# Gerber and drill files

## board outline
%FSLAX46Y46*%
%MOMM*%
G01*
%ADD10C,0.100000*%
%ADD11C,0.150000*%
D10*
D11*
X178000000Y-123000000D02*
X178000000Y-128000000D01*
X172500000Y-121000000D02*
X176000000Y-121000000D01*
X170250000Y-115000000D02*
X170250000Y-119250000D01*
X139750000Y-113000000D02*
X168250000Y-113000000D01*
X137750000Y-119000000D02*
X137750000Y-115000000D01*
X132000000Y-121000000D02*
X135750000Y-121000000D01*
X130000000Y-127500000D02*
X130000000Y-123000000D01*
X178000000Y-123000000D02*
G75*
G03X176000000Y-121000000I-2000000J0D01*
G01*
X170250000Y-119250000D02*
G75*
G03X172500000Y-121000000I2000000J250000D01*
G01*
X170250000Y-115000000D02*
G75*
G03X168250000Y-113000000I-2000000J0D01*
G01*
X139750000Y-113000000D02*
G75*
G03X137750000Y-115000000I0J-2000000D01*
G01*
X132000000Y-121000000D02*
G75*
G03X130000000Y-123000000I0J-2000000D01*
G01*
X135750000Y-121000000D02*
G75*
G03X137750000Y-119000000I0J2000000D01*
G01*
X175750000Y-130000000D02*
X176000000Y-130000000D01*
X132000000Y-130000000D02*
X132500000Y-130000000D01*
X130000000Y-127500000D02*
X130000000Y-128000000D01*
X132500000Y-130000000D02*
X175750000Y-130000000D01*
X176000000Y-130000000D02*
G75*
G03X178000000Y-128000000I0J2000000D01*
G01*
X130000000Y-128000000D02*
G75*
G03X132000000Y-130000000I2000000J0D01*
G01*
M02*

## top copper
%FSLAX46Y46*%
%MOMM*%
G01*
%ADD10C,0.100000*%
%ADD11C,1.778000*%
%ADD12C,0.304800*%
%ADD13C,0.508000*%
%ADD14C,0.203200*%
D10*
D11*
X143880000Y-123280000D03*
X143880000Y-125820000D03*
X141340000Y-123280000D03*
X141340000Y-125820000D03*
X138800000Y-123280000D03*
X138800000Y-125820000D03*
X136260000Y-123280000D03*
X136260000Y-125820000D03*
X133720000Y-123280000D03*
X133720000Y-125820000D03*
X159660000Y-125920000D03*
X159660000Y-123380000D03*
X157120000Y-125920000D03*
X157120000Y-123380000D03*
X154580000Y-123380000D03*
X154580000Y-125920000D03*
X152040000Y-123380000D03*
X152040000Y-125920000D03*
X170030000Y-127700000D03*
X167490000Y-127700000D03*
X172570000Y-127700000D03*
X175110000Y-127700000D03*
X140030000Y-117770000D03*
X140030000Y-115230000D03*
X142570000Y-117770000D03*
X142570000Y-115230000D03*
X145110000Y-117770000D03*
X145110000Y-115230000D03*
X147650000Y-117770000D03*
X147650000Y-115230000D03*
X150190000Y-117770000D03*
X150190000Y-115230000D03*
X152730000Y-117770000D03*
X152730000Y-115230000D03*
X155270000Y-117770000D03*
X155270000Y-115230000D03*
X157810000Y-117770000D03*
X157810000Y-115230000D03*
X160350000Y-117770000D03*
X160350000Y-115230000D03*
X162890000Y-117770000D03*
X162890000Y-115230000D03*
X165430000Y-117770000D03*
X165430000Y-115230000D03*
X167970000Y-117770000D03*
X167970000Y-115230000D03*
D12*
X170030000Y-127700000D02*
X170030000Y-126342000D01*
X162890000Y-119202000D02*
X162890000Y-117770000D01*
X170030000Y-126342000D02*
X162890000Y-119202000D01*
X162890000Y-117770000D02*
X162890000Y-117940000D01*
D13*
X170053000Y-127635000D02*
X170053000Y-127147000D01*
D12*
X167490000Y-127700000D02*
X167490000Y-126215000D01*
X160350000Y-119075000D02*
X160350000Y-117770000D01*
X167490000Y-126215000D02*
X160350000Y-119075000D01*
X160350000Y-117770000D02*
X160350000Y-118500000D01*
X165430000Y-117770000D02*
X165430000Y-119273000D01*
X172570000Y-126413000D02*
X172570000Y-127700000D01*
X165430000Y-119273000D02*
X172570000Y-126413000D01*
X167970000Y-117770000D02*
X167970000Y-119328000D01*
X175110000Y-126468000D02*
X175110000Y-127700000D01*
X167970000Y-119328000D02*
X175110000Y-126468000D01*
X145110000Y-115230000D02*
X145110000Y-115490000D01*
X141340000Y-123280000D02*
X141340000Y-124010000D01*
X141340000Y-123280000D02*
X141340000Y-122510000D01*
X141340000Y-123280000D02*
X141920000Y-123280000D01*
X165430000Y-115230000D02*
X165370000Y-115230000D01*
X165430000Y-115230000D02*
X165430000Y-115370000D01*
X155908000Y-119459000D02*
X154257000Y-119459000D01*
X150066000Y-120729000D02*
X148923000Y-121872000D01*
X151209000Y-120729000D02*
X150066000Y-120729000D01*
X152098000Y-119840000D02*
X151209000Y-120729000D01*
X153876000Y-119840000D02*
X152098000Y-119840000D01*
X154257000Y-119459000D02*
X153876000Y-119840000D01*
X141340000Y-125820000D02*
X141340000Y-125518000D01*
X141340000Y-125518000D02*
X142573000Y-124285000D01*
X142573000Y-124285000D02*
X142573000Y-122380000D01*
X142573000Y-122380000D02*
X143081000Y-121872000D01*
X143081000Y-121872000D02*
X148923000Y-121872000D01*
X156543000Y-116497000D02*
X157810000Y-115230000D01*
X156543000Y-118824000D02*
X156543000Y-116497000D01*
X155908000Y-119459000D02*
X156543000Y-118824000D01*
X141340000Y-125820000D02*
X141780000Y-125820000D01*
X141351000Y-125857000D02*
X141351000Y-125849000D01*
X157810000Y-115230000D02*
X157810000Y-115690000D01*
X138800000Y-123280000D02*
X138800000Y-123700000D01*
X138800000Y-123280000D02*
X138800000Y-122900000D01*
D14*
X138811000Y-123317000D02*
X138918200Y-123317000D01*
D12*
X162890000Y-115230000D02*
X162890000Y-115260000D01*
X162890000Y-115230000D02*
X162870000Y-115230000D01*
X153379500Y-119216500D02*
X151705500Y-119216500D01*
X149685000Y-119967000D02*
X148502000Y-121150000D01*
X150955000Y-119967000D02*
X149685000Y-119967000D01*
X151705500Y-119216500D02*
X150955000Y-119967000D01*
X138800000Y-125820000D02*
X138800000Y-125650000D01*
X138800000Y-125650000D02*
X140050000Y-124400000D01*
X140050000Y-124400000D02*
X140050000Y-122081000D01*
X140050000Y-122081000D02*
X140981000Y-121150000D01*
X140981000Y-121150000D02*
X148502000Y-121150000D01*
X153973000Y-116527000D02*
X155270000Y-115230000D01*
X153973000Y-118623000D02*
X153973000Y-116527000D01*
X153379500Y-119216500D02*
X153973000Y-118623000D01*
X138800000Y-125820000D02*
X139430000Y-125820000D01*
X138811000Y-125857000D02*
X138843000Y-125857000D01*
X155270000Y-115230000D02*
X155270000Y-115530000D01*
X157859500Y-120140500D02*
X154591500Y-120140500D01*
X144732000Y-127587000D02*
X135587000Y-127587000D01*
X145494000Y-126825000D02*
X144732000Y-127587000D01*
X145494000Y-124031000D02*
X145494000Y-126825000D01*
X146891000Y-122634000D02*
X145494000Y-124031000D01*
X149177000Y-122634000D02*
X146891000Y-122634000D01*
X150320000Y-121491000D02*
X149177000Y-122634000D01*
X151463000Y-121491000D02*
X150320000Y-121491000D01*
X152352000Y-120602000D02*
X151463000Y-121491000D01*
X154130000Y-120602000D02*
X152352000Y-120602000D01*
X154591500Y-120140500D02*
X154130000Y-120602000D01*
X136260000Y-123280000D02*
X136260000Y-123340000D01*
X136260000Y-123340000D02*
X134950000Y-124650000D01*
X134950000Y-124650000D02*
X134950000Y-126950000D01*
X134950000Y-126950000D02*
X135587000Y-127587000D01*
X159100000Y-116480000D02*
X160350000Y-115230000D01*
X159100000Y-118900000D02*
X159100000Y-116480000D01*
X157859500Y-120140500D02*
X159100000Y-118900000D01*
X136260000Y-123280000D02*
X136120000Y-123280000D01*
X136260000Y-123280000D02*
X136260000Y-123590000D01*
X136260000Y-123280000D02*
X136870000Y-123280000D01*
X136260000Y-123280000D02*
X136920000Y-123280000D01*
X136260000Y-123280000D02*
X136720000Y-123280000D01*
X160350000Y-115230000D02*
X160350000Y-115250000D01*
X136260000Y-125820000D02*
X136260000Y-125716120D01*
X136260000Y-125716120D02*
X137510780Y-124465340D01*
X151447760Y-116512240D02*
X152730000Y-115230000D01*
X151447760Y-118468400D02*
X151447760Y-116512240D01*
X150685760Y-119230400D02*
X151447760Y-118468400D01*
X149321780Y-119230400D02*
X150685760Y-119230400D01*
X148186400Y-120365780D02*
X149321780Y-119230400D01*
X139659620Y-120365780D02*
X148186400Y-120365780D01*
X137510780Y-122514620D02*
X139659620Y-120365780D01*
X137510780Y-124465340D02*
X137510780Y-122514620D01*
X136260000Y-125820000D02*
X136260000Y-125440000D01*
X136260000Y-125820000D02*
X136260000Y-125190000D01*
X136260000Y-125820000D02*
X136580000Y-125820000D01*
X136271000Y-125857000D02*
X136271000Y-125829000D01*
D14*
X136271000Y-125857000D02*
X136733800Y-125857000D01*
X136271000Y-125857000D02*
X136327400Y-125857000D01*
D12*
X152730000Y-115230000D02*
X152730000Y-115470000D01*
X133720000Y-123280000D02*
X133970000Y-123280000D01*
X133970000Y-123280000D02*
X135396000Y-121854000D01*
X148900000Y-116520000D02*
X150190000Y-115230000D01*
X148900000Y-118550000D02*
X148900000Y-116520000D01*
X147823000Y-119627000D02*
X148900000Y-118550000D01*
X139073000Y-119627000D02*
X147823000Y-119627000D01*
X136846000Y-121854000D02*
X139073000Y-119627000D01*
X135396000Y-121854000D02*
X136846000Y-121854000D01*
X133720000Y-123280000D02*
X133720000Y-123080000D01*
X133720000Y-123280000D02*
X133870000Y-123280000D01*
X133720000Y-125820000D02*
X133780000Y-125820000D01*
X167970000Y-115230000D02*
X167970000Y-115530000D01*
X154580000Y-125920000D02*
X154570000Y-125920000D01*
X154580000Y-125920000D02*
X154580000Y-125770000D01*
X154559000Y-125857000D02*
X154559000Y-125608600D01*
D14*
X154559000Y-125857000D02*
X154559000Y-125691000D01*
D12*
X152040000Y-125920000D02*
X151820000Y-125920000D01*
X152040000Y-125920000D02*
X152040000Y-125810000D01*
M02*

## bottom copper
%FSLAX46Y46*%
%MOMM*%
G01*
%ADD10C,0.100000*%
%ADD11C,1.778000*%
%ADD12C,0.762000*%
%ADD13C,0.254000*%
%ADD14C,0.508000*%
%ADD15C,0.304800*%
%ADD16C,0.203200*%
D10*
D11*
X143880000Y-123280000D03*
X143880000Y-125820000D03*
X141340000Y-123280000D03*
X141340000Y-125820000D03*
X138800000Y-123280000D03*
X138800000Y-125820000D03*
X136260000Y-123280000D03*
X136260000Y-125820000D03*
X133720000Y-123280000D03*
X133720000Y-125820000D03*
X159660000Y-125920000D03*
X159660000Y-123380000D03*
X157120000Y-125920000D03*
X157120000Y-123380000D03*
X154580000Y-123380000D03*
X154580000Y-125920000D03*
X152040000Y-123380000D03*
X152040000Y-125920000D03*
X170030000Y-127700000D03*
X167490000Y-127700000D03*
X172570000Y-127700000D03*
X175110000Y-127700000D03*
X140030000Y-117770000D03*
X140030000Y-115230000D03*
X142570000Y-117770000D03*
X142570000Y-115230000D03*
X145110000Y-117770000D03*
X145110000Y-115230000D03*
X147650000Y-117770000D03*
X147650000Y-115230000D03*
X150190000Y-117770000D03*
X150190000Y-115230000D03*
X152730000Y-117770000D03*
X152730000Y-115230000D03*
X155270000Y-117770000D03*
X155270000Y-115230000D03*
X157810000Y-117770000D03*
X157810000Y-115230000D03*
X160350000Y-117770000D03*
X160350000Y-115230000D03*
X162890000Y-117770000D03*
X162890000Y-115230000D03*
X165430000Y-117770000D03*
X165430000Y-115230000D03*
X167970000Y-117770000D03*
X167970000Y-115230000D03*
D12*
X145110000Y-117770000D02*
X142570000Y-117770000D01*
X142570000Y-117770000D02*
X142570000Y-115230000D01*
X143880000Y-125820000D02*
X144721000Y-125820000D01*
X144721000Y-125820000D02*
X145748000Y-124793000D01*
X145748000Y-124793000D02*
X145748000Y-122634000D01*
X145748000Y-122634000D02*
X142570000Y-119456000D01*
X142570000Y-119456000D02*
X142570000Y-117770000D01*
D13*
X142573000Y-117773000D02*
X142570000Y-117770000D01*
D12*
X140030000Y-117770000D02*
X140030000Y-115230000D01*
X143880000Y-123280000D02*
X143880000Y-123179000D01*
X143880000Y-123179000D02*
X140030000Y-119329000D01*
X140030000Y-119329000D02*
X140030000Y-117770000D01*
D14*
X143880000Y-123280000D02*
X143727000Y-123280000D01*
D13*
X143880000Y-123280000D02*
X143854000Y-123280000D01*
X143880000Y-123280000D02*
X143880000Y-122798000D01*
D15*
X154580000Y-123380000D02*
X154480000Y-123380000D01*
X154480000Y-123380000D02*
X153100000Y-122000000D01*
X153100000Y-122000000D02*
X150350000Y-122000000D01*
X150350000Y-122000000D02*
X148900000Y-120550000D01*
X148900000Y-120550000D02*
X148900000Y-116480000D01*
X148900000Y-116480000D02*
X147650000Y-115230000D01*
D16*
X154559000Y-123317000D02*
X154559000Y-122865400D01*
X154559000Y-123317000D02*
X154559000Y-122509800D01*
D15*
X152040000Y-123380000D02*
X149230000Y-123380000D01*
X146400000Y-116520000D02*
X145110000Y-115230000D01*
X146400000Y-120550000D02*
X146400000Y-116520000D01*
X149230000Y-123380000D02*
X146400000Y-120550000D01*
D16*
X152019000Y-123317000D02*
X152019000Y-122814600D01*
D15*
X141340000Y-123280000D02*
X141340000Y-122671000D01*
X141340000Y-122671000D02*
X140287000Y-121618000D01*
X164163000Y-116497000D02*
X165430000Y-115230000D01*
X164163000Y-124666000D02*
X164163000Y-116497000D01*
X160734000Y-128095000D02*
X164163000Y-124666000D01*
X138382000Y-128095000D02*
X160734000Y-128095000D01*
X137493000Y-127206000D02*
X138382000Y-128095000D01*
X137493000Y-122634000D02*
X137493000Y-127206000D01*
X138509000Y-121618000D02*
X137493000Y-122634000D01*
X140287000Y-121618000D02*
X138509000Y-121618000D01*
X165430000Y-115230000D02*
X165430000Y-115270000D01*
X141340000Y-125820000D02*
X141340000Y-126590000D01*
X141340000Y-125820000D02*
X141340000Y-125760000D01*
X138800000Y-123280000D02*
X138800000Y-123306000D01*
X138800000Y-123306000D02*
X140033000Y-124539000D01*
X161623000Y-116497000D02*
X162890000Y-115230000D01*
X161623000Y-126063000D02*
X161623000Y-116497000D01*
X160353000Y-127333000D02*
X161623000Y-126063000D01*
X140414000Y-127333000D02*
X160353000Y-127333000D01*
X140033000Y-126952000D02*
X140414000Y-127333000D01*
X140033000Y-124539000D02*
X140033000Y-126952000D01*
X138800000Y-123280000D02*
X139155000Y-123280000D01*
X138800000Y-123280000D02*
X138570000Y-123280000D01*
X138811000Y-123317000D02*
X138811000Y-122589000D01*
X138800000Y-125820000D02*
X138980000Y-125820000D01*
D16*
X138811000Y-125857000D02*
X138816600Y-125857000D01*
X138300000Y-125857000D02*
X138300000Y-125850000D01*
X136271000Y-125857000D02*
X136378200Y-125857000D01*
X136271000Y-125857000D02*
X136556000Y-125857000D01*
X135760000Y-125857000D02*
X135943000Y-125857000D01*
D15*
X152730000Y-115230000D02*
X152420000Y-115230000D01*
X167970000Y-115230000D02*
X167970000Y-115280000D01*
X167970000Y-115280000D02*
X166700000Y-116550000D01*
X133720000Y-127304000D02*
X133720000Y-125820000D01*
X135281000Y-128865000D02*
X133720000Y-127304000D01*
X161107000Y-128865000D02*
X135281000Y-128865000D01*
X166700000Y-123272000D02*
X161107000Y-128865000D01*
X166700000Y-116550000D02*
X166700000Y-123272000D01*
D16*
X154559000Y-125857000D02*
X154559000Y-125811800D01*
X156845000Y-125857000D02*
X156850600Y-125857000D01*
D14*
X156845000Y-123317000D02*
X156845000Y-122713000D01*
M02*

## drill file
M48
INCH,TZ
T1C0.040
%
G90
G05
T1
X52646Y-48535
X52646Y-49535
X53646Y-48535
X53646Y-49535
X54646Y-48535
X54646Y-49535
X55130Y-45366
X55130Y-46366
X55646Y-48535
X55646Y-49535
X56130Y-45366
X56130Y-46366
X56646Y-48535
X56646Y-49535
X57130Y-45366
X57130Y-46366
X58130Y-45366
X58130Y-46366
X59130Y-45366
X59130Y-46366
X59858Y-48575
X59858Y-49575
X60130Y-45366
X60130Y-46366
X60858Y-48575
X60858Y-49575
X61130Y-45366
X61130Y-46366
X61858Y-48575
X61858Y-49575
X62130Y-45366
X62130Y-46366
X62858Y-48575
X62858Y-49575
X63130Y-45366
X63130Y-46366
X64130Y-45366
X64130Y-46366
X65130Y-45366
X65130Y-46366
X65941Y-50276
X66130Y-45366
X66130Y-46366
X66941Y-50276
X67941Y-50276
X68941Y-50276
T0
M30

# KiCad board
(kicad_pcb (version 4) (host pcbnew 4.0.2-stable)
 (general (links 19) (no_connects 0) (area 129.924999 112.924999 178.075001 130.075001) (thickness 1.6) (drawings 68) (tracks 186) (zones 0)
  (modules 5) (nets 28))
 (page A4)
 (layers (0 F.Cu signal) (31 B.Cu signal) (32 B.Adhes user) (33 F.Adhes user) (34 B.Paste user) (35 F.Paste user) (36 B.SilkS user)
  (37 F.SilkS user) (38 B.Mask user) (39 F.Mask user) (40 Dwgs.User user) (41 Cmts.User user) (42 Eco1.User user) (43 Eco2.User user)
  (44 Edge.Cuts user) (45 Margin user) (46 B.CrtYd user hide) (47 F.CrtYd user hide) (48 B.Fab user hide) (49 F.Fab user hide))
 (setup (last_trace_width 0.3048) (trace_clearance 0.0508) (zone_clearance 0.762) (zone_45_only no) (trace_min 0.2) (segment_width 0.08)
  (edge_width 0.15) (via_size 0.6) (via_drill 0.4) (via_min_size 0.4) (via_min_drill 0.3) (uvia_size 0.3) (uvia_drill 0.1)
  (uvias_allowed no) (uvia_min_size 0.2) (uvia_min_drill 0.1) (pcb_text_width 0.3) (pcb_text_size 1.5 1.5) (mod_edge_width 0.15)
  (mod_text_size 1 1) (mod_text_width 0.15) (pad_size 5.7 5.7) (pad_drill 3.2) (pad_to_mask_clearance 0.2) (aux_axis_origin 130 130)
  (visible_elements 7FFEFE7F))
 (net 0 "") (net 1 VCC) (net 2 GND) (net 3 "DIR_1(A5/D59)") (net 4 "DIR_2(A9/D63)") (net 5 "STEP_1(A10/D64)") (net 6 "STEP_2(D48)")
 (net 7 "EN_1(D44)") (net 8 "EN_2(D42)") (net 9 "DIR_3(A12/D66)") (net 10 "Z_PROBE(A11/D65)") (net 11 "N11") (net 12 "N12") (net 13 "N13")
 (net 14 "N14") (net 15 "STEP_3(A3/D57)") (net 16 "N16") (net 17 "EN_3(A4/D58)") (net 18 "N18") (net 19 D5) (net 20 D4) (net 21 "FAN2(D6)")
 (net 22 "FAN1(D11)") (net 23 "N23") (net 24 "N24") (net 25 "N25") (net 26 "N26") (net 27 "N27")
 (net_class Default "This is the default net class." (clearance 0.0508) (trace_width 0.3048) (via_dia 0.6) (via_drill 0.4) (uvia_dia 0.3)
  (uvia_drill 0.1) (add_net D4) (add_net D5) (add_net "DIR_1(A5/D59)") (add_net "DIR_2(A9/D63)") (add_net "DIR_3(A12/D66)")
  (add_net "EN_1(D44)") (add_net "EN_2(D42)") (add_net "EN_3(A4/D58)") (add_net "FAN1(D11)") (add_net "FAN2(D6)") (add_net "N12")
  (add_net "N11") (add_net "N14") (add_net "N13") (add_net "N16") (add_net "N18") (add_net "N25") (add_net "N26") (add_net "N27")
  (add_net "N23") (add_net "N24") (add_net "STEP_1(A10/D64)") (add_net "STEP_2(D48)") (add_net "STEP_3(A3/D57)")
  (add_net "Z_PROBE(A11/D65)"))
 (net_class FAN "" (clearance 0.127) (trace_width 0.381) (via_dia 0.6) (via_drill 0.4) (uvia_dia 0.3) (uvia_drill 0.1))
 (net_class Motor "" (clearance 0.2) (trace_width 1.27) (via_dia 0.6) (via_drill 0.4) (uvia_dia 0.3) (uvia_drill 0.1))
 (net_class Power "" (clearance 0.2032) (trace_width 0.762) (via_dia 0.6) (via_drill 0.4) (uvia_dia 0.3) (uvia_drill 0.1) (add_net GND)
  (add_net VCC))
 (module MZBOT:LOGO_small (layer F.Cu) (at 167.66058 124.78538)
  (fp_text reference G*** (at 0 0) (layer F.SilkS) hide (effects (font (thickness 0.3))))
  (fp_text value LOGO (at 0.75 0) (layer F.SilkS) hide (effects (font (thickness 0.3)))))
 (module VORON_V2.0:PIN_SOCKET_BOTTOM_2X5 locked (layer F.Cu) (at 138.8 124.55 180)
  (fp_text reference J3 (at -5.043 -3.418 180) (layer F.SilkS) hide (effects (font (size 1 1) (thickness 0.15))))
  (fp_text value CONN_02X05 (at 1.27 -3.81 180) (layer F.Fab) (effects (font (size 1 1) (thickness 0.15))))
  (pad 1 thru_hole circle (at -5.08 1.27 180) (size 1.778 1.778) (drill 1.016) (layers *.Cu *.Mask F.SilkS) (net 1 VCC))
  (pad 2 thru_hole circle (at -5.08 -1.27 180) (size 1.778 1.778) (drill 1.016) (layers *.Cu *.Mask F.SilkS) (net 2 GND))
  (pad 3 thru_hole circle (at -2.54 1.27 180) (size 1.778 1.778) (drill 1.016) (layers *.Cu *.Mask F.SilkS) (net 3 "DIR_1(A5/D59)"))
  (pad 4 thru_hole circle (at -2.54 -1.27 180) (size 1.778 1.778) (drill 1.016) (layers *.Cu *.Mask F.SilkS) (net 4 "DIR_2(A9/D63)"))
  (pad 5 thru_hole circle (at 0 1.27 180) (size 1.778 1.778) (drill 1.016) (layers *.Cu *.Mask F.SilkS) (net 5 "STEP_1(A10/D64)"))
  (pad 6 thru_hole circle (at 0 -1.27 180) (size 1.778 1.778) (drill 1.016) (layers *.Cu *.Mask F.SilkS) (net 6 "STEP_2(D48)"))
  (pad 7 thru_hole circle (at 2.54 1.27 180) (size 1.778 1.778) (drill 1.016) (layers *.Cu *.Mask F.SilkS) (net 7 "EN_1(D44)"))
  (pad 8 thru_hole circle (at 2.54 -1.27 180) (size 1.778 1.778) (drill 1.016) (layers *.Cu *.Mask F.SilkS) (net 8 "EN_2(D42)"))
  (pad 9 thru_hole circle (at 5.08 1.27 180) (size 1.778 1.778) (drill 1.016) (layers *.Cu *.Mask F.SilkS) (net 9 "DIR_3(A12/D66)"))
  (pad 10 thru_hole circle (at 5.08 -1.27 180) (size 1.778 1.778) (drill 1.016) (layers *.Cu *.Mask F.SilkS) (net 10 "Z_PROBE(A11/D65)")))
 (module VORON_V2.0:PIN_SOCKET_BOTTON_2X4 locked (layer F.Cu) (at 155.85 124.65 180)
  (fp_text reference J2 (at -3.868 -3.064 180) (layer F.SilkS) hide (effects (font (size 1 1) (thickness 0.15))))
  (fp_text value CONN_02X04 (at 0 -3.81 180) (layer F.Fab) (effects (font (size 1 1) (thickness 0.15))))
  (pad 2 thru_hole circle (at -3.81 -1.27 180) (size 1.778 1.778) (drill 1.016) (layers *.Cu *.Mask F.SilkS) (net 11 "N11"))
  (pad 1 thru_hole circle (at -3.81 1.27 180) (size 1.778 1.778) (drill 1.016) (layers *.Cu *.Mask F.SilkS) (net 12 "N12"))
  (pad 4 thru_hole circle (at -1.27 -1.27 180) (size 1.778 1.778) (drill 1.016) (layers *.Cu *.Mask F.SilkS) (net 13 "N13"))
  (pad 3 thru_hole circle (at -1.27 1.27 180) (size 1.778 1.778) (drill 1.016) (layers *.Cu *.Mask F.SilkS) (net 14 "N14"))
  (pad 5 thru_hole circle (at 1.27 1.27 180) (size 1.778 1.778) (drill 1.016) (layers *.Cu *.Mask F.SilkS) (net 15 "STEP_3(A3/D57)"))
  (pad 6 thru_hole circle (at 1.27 -1.27 180) (size 1.778 1.778) (drill 1.016) (layers *.Cu *.Mask F.SilkS) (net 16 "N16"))
  (pad 7 thru_hole circle (at 3.81 1.27 180) (size 1.778 1.778) (drill 1.016) (layers *.Cu *.Mask F.SilkS) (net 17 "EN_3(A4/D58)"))
  (pad 8 thru_hole circle (at 3.81 -1.27 180) (size 1.778 1.778) (drill 1.016) (layers *.Cu *.Mask F.SilkS) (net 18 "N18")))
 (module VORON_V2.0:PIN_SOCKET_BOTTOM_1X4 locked (layer F.Cu) (at 171.3 127.7)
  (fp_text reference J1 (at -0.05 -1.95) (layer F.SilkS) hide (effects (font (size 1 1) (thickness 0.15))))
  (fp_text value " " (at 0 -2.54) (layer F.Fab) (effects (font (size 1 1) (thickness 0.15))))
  (pad 2 thru_hole circle (at -1.27 0) (size 1.778 1.778) (drill 1.016) (layers *.Cu *.Mask F.SilkS) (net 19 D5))
  (pad 1 thru_hole circle (at -3.81 0) (size 1.778 1.778) (drill 1.016) (layers *.Cu *.Mask F.SilkS) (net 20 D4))
  (pad 3 thru_hole circle (at 1.27 0) (size 1.778 1.778) (drill 1.016) (layers *.Cu *.Mask F.SilkS) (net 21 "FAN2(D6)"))
  (pad 4 thru_hole circle (at 3.81 0) (size 1.778 1.778) (drill 1.016) (layers *.Cu *.Mask F.SilkS) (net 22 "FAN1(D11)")))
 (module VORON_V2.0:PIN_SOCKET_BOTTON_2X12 (layer F.Cu) (at 154 116.5)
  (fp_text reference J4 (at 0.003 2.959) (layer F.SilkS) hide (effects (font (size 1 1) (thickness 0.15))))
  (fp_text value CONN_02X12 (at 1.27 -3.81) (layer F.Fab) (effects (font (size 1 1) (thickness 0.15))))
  (pad 1 thru_hole circle (at -13.97 1.27) (size 1.778 1.778) (drill 1.016) (layers *.Cu *.Mask F.SilkS) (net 1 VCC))
  (pad 2 thru_hole circle (at -13.97 -1.27) (size 1.778 1.778) (drill 1.016) (layers *.Cu *.Mask F.SilkS) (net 1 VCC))
  (pad 3 thru_hole circle (at -11.43 1.27) (size 1.778 1.778) (drill 1.016) (layers *.Cu *.Mask F.SilkS) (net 2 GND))
  (pad 4 thru_hole circle (at -11.43 -1.27) (size 1.778 1.778) (drill 1.016) (layers *.Cu *.Mask F.SilkS) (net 2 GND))
  (pad 5 thru_hole circle (at -8.89 1.27) (size 1.778 1.778) (drill 1.016) (layers *.Cu *.Mask F.SilkS) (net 2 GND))
  (pad 6 thru_hole circle (at -8.89 -1.27) (size 1.778 1.778) (drill 1.016) (layers *.Cu *.Mask F.SilkS) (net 17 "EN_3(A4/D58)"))
  (pad 7 thru_hole circle (at -6.35 1.27) (size 1.778 1.778) (drill 1.016) (layers *.Cu *.Mask F.SilkS) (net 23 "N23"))
  (pad 8 thru_hole circle (at -6.35 -1.27) (size 1.778 1.778) (drill 1.016) (layers *.Cu *.Mask F.SilkS) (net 15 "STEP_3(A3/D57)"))
  (pad 9 thru_hole circle (at -3.81 1.27) (size 1.778 1.778) (drill 1.016) (layers *.Cu *.Mask F.SilkS) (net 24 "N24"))
  (pad 10 thru_hole circle (at -3.81 -1.27) (size 1.778 1.778) (drill 1.016) (layers *.Cu *.Mask F.SilkS) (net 9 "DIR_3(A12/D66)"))
  (pad 11 thru_hole circle (at -1.27 1.27) (size 1.778 1.778) (drill 1.016) (layers *.Cu *.Mask F.SilkS) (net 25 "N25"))
  (pad 12 thru_hole circle (at -1.27 -1.27) (size 1.778 1.778) (drill 1.016) (layers *.Cu *.Mask F.SilkS) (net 8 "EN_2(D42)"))
  (pad 13 thru_hole circle (at 1.27 1.27) (size 1.778 1.778) (drill 1.016) (layers *.Cu *.Mask F.SilkS) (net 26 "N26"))
  (pad 14 thru_hole circle (at 1.27 -1.27) (size 1.778 1.778) (drill 1.016) (layers *.Cu *.Mask F.SilkS) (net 6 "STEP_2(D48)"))
  (pad 15 thru_hole circle (at 3.81 1.27) (size 1.778 1.778) (drill 1.016) (layers *.Cu *.Mask F.SilkS) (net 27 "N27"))
  (pad 16 thru_hole circle (at 3.81 -1.27) (size 1.778 1.778) (drill 1.016) (layers *.Cu *.Mask F.SilkS) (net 4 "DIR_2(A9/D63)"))
  (pad 17 thru_hole circle (at 6.35 1.27) (size 1.778 1.778) (drill 1.016) (layers *.Cu *.Mask F.SilkS) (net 20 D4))
  (pad 18 thru_hole circle (at 6.35 -1.27) (size 1.778 1.778) (drill 1.016) (layers *.Cu *.Mask F.SilkS) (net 7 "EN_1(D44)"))
  (pad 19 thru_hole circle (at 8.89 1.27) (size 1.778 1.778) (drill 1.016) (layers *.Cu *.Mask F.SilkS) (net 19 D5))
  (pad 20 thru_hole circle (at 8.89 -1.27) (size 1.778 1.778) (drill 1.016) (layers *.Cu *.Mask F.SilkS) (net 5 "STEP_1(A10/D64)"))
  (pad 21 thru_hole circle (at 11.43 1.27) (size 1.778 1.778) (drill 1.016) (layers *.Cu *.Mask F.SilkS) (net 21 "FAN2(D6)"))
  (pad 22 thru_hole circle (at 11.43 -1.27) (size 1.778 1.778) (drill 1.016) (layers *.Cu *.Mask F.SilkS) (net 3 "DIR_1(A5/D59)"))
  (pad 23 thru_hole circle (at 13.97 1.27) (size 1.778 1.778) (drill 1.016) (layers *.Cu *.Mask F.SilkS) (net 22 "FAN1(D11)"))
  (pad 24 thru_hole circle (at 13.97 -1.27) (size 1.778 1.778) (drill 1.016) (layers *.Cu *.Mask F.SilkS) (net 10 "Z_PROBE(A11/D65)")))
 (gr_line (start 178 123) (end 178 128) (angle 90) (layer Edge.Cuts) (width 0.15))
 (gr_line (start 172.5 121) (end 176 121) (angle 90) (layer Edge.Cuts) (width 0.15))
 (gr_line (start 170.25 115) (end 170.25 119.25) (angle 90) (layer Edge.Cuts) (width 0.15))
 (gr_line (start 139.75 113) (end 168.25 113) (angle 90) (layer Edge.Cuts) (width 0.15))
 (gr_line (start 137.75 119) (end 137.75 115) (angle 90) (layer Edge.Cuts) (width 0.15))
 (gr_line (start 132 121) (end 135.75 121) (angle 90) (layer Edge.Cuts) (width 0.15))
 (gr_line (start 130 127.5) (end 130 123) (angle 90) (layer Edge.Cuts) (width 0.15))
 (gr_arc (start 176 123) (end 176 121) (angle 90) (layer Edge.Cuts) (width 0.15))
 (gr_arc (start 172.25 119) (end 172.5 121) (angle 90) (layer Edge.Cuts) (width 0.15))
 (gr_arc (start 168.25 115) (end 168.25 113) (angle 90) (layer Edge.Cuts) (width 0.15))
 (gr_arc (start 139.75 115) (end 137.75 115) (angle 90) (layer Edge.Cuts) (width 0.15))
 (gr_arc (start 132 123) (end 130 123) (angle 90) (layer Edge.Cuts) (width 0.15))
 (gr_arc (start 135.75 119) (end 137.75 119) (angle 90) (layer Edge.Cuts) (width 0.15))
 (gr_line (start 175.75 130) (end 176 130) (angle 90) (layer Edge.Cuts) (width 0.15))
 (gr_line (start 132 130) (end 132.5 130) (angle 90) (layer Edge.Cuts) (width 0.15))
 (gr_line (start 130 127.5) (end 130 128) (angle 90) (layer Edge.Cuts) (width 0.15))
 (gr_line (start 132.5 130) (end 175.75 130) (angle 90) (layer Edge.Cuts) (width 0.15))
 (gr_arc (start 176 128) (end 178 128) (angle 90) (layer Edge.Cuts) (width 0.15))
 (gr_arc (start 132 128) (end 132 130) (angle 90) (layer Edge.Cuts) (width 0.15))
 (segment (start 145.11 117.77) (end 142.57 117.77) (width 0.762) (layer B.Cu) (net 2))
 (segment (start 142.57 117.77) (end 142.57 115.23) (width 0.762) (layer B.Cu) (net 2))
 (segment (start 143.88 125.82) (end 144.721 125.82) (width 0.762) (layer B.Cu) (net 2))
 (segment (start 144.721 125.82) (end 145.748 124.793) (width 0.762) (layer B.Cu) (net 2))
 (segment (start 145.748 124.793) (end 145.748 122.634) (width 0.762) (layer B.Cu) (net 2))
 (segment (start 145.748 122.634) (end 142.57 119.456) (width 0.762) (layer B.Cu) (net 2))
 (segment (start 142.57 119.456) (end 142.57 117.77) (width 0.762) (layer B.Cu) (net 2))
 (segment (start 142.573 117.773) (end 142.57 117.77) (width 0.254) (layer B.Cu) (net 2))
 (segment (start 140.03 117.77) (end 140.03 115.23) (width 0.762) (layer B.Cu) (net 1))
 (segment (start 143.88 123.28) (end 143.88 123.179) (width 0.762) (layer B.Cu) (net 1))
 (segment (start 143.88 123.179) (end 140.03 119.329) (width 0.762) (layer B.Cu) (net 1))
 (segment (start 140.03 119.329) (end 140.03 117.77) (width 0.762) (layer B.Cu) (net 1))
 (segment (start 143.88 123.28) (end 143.727 123.28) (width 0.508) (layer B.Cu) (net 1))
 (segment (start 143.88 123.28) (end 143.854 123.28) (width 0.254) (layer B.Cu) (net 1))
 (segment (start 143.88 123.28) (end 143.88 122.798) (width 0.254) (layer B.Cu) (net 1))
 (segment (start 170.03 127.7) (end 170.03 126.342) (width 0.3048) (layer F.Cu) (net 19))
 (segment (start 162.89 119.202) (end 162.89 117.77) (width 0.3048) (layer F.Cu) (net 19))
 (segment (start 170.03 126.342) (end 162.89 119.202) (width 0.3048) (layer F.Cu) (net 19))
 (segment (start 162.89 117.77) (end 162.89 117.94) (width 0.3048) (layer F.Cu) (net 19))
 (segment (start 170.053 127.635) (end 170.053 127.147) (width 0.508) (layer F.Cu) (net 19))
 (segment (start 167.49 127.7) (end 167.49 126.215) (width 0.3048) (layer F.Cu) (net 20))
 (segment (start 160.35 119.075) (end 160.35 117.77) (width 0.3048) (layer F.Cu) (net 20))
 (segment (start 167.49 126.215) (end 160.35 119.075) (width 0.3048) (layer F.Cu) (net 20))
 (segment (start 160.35 117.77) (end 160.35 118.5) (width 0.3048) (layer F.Cu) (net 20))
 (segment (start 165.43 117.77) (end 165.43 119.273) (width 0.3048) (layer F.Cu) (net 21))
 (segment (start 172.57 126.413) (end 172.57 127.7) (width 0.3048) (layer F.Cu) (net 21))
 (segment (start 165.43 119.273) (end 172.57 126.413) (width 0.3048) (layer F.Cu) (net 21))
 (segment (start 167.97 117.77) (end 167.97 119.328) (width 0.3048) (layer F.Cu) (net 22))
 (segment (start 175.11 126.468) (end 175.11 127.7) (width 0.3048) (layer F.Cu) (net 22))
 (segment (start 167.97 119.328) (end 175.11 126.468) (width 0.3048) (layer F.Cu) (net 22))
 (segment (start 154.58 123.38) (end 154.48 123.38) (width 0.3048) (layer B.Cu) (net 15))
 (segment (start 154.48 123.38) (end 153.1 122) (width 0.3048) (layer B.Cu) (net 15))
 (segment (start 153.1 122) (end 150.35 122) (width 0.3048) (layer B.Cu) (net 15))
 (segment (start 150.35 122) (end 148.9 120.55) (width 0.3048) (layer B.Cu) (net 15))
 (segment (start 148.9 120.55) (end 148.9 116.48) (width 0.3048) (layer B.Cu) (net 15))
 (segment (start 148.9 116.48) (end 147.65 115.23) (width 0.3048) (layer B.Cu) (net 15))
 (segment (start 154.559 123.317) (end 154.559 122.8654) (width 0.2032) (layer B.Cu) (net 15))
 (segment (start 154.559 123.317) (end 154.559 122.5098) (width 0.2032) (layer B.Cu) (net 15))
 (segment (start 152.04 123.38) (end 149.23 123.38) (width 0.3048) (layer B.Cu) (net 17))
 (segment (start 146.4 116.52) (end 145.11 115.23) (width 0.3048) (layer B.Cu) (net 17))
 (segment (start 146.4 120.55) (end 146.4 116.52) (width 0.3048) (layer B.Cu) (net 17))
 (segment (start 149.23 123.38) (end 146.4 120.55) (width 0.3048) (layer B.Cu) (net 17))
 (segment (start 152.019 123.317) (end 152.019 122.8146) (width 0.2032) (layer B.Cu) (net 17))
 (segment (start 145.11 115.23) (end 145.11 115.49) (width 0.3048) (layer F.Cu) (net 17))
 (segment (start 141.34 123.28) (end 141.34 122.671) (width 0.3048) (layer B.Cu) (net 3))
 (segment (start 141.34 122.671) (end 140.287 121.618) (width 0.3048) (layer B.Cu) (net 3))
 (segment (start 164.163 116.497) (end 165.43 115.23) (width 0.3048) (layer B.Cu) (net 3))
 (segment (start 164.163 124.666) (end 164.163 116.497) (width 0.3048) (layer B.Cu) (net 3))
 (segment (start 160.734 128.095) (end 164.163 124.666) (width 0.3048) (layer B.Cu) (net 3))
 (segment (start 138.382 128.095) (end 160.734 128.095) (width 0.3048) (layer B.Cu) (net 3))
 (segment (start 137.493 127.206) (end 138.382 128.095) (width 0.3048) (layer B.Cu) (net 3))
 (segment (start 137.493 122.634) (end 137.493 127.206) (width 0.3048) (layer B.Cu) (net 3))
 (segment (start 138.509 121.618) (end 137.493 122.634) (width 0.3048) (layer B.Cu) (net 3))
 (segment (start 140.287 121.618) (end 138.509 121.618) (width 0.3048) (layer B.Cu) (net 3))
 (segment (start 165.43 115.23) (end 165.43 115.27) (width 0.3048) (layer B.Cu) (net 3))
 (segment (start 141.34 123.28) (end 141.34 124.01) (width 0.3048) (layer F.Cu) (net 3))
 (segment (start 141.34 123.28) (end 141.34 122.51) (width 0.3048) (layer F.Cu) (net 3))
 (segment (start 141.34 123.28) (end 141.92 123.28) (width 0.3048) (layer F.Cu) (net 3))
 (segment (start 165.43 115.23) (end 165.37 115.23) (width 0.3048) (layer F.Cu) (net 3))
 (segment (start 165.43 115.23) (end 165.43 115.37) (width 0.3048) (layer F.Cu) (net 3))
 (segment (start 155.908 119.459) (end 154.257 119.459) (width 0.3048) (layer F.Cu) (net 4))
 (segment (start 150.066 120.729) (end 148.923 121.872) (width 0.3048) (layer F.Cu) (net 4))
 (segment (start 151.209 120.729) (end 150.066 120.729) (width 0.3048) (layer F.Cu) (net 4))
 (segment (start 152.098 119.84) (end 151.209 120.729) (width 0.3048) (layer F.Cu) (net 4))
 (segment (start 153.876 119.84) (end 152.098 119.84) (width 0.3048) (layer F.Cu) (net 4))
 (segment (start 154.257 119.459) (end 153.876 119.84) (width 0.3048) (layer F.Cu) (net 4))
 (segment (start 141.34 125.82) (end 141.34 125.518) (width 0.3048) (layer F.Cu) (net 4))
 (segment (start 141.34 125.518) (end 142.573 124.285) (width 0.3048) (layer F.Cu) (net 4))
 (segment (start 142.573 124.285) (end 142.573 122.38) (width 0.3048) (layer F.Cu) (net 4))
 (segment (start 142.573 122.38) (end 143.081 121.872) (width 0.3048) (layer F.Cu) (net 4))
 (segment (start 143.081 121.872) (end 148.923 121.872) (width 0.3048) (layer F.Cu) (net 4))
 (segment (start 156.543 116.497) (end 157.81 115.23) (width 0.3048) (layer F.Cu) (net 4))
 (segment (start 156.543 118.824) (end 156.543 116.497) (width 0.3048) (layer F.Cu) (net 4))
 (segment (start 155.908 119.459) (end 156.543 118.824) (width 0.3048) (layer F.Cu) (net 4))
 (segment (start 141.34 125.82) (end 141.34 126.59) (width 0.3048) (layer B.Cu) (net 4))
 (segment (start 141.34 125.82) (end 141.34 125.76) (width 0.3048) (layer B.Cu) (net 4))
 (segment (start 141.34 125.82) (end 141.78 125.82) (width 0.3048) (layer F.Cu) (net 4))
 (segment (start 141.351 125.857) (end 141.351 125.849) (width 0.3048) (layer F.Cu) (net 4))
 (segment (start 157.81 115.23) (end 157.81 115.69) (width 0.3048) (layer F.Cu) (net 4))
 (segment (start 138.8 123.28) (end 138.8 123.306) (width 0.3048) (layer B.Cu) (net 5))
 (segment (start 138.8 123.306) (end 140.033 124.539) (width 0.3048) (layer B.Cu) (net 5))
 (segment (start 161.623 116.497) (end 162.89 115.23) (width 0.3048) (layer B.Cu) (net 5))
 (segment (start 161.623 126.063) (end 161.623 116.497) (width 0.3048) (layer B.Cu) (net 5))
 (segment (start 160.353 127.333) (end 161.623 126.063) (width 0.3048) (layer B.Cu) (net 5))
 (segment (start 140.414 127.333) (end 160.353 127.333) (width 0.3048) (layer B.Cu) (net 5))
 (segment (start 140.033 126.952) (end 140.414 127.333) (width 0.3048) (layer B.Cu) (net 5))
 (segment (start 140.033 124.539) (end 140.033 126.952) (width 0.3048) (layer B.Cu) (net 5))
 (segment (start 138.8 123.28) (end 139.155 123.28) (width 0.3048) (layer B.Cu) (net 5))
 (segment (start 138.8 123.28) (end 138.57 123.28) (width 0.3048) (layer B.Cu) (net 5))
 (segment (start 138.8 123.28) (end 138.8 123.7) (width 0.3048) (layer F.Cu) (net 5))
 (segment (start 138.8 123.28) (end 138.8 122.9) (width 0.3048) (layer F.Cu) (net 5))
 (segment (start 138.811 123.317) (end 138.9182 123.317) (width 0.2032) (layer F.Cu) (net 5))
 (segment (start 138.811 123.317) (end 138.811 122.589) (width 0.3048) (layer B.Cu) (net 5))
 (segment (start 162.89 115.23) (end 162.89 115.26) (width 0.3048) (layer F.Cu) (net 5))
 (segment (start 162.89 115.23) (end 162.87 115.23) (width 0.3048) (layer F.Cu) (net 5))
 (segment (start 153.3795 119.2165) (end 151.7055 119.2165) (width 0.3048) (layer F.Cu) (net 6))
 (segment (start 149.685 119.967) (end 148.502 121.15) (width 0.3048) (layer F.Cu) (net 6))
 (segment (start 150.955 119.967) (end 149.685 119.967) (width 0.3048) (layer F.Cu) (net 6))
 (segment (start 151.7055 119.2165) (end 150.955 119.967) (width 0.3048) (layer F.Cu) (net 6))
 (segment (start 138.8 125.82) (end 138.8 125.65) (width 0.3048) (layer F.Cu) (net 6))
 (segment (start 138.8 125.65) (end 140.05 124.4) (width 0.3048) (layer F.Cu) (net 6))
 (segment (start 140.05 124.4) (end 140.05 122.081) (width 0.3048) (layer F.Cu) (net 6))
 (segment (start 140.05 122.081) (end 140.981 121.15) (width 0.3048) (layer F.Cu) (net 6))
 (segment (start 140.981 121.15) (end 148.502 121.15) (width 0.3048) (layer F.Cu) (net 6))
 (segment (start 153.973 116.527) (end 155.27 115.23) (width 0.3048) (layer F.Cu) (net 6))
 (segment (start 153.973 118.623) (end 153.973 116.527) (width 0.3048) (layer F.Cu) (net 6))
 (segment (start 153.3795 119.2165) (end 153.973 118.623) (width 0.3048) (layer F.Cu) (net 6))
 (segment (start 138.8 125.82) (end 139.43 125.82) (width 0.3048) (layer F.Cu) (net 6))
 (segment (start 138.8 125.82) (end 138.98 125.82) (width 0.3048) (layer B.Cu) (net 6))
 (segment (start 138.811 125.857) (end 138.8166 125.857) (width 0.2032) (layer B.Cu) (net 6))
 (segment (start 138.3 125.857) (end 138.3 125.85) (width 0.2032) (layer B.Cu) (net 6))
 (segment (start 138.811 125.857) (end 138.843 125.857) (width 0.3048) (layer F.Cu) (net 6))
 (segment (start 155.27 115.23) (end 155.27 115.53) (width 0.3048) (layer F.Cu) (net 6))
 (segment (start 157.8595 120.1405) (end 154.5915 120.1405) (width 0.3048) (layer F.Cu) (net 7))
 (segment (start 144.732 127.587) (end 135.587 127.587) (width 0.3048) (layer F.Cu) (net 7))
 (segment (start 145.494 126.825) (end 144.732 127.587) (width 0.3048) (layer F.Cu) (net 7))
 (segment (start 145.494 124.031) (end 145.494 126.825) (width 0.3048) (layer F.Cu) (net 7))
 (segment (start 146.891 122.634) (end 145.494 124.031) (width 0.3048) (layer F.Cu) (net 7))
 (segment (start 149.177 122.634) (end 146.891 122.634) (width 0.3048) (layer F.Cu) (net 7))
 (segment (start 150.32 121.491) (end 149.177 122.634) (width 0.3048) (layer F.Cu) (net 7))
 (segment (start 151.463 121.491) (end 150.32 121.491) (width 0.3048) (layer F.Cu) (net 7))
 (segment (start 152.352 120.602) (end 151.463 121.491) (width 0.3048) (layer F.Cu) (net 7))
 (segment (start 154.13 120.602) (end 152.352 120.602) (width 0.3048) (layer F.Cu) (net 7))
 (segment (start 154.5915 120.1405) (end 154.13 120.602) (width 0.3048) (layer F.Cu) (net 7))
 (segment (start 136.26 123.28) (end 136.26 123.34) (width 0.3048) (layer F.Cu) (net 7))
 (segment (start 136.26 123.34) (end 134.95 124.65) (width 0.3048) (layer F.Cu) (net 7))
 (segment (start 134.95 124.65) (end 134.95 126.95) (width 0.3048) (layer F.Cu) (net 7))
 (segment (start 134.95 126.95) (end 135.587 127.587) (width 0.3048) (layer F.Cu) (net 7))
 (segment (start 159.1 116.48) (end 160.35 115.23) (width 0.3048) (layer F.Cu) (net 7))
 (segment (start 159.1 118.9) (end 159.1 116.48) (width 0.3048) (layer F.Cu) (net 7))
 (segment (start 157.8595 120.1405) (end 159.1 118.9) (width 0.3048) (layer F.Cu) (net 7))
 (segment (start 136.26 123.28) (end 136.12 123.28) (width 0.3048) (layer F.Cu) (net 7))
 (segment (start 136.26 123.28) (end 136.26 123.59) (width 0.3048) (layer F.Cu) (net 7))
 (segment (start 136.26 123.28) (end 136.87 123.28) (width 0.3048) (layer F.Cu) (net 7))
 (segment (start 136.26 123.28) (end 136.92 123.28) (width 0.3048) (layer F.Cu) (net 7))
 (segment (start 136.26 123.28) (end 136.72 123.28) (width 0.3048) (layer F.Cu) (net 7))
 (segment (start 160.35 115.23) (end 160.35 115.25) (width 0.3048) (layer F.Cu) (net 7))
 (segment (start 136.26 125.82) (end 136.26 125.71612) (width 0.3048) (layer F.Cu) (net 8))
 (segment (start 136.26 125.71612) (end 137.51078 124.46534) (width 0.3048) (layer F.Cu) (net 8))
 (segment (start 151.44776 116.51224) (end 152.73 115.23) (width 0.3048) (layer F.Cu) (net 8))
 (segment (start 151.44776 118.4684) (end 151.44776 116.51224) (width 0.3048) (layer F.Cu) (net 8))
 (segment (start 150.68576 119.2304) (end 151.44776 118.4684) (width 0.3048) (layer F.Cu) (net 8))
 (segment (start 149.32178 119.2304) (end 150.68576 119.2304) (width 0.3048) (layer F.Cu) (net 8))
 (segment (start 148.1864 120.36578) (end 149.32178 119.2304) (width 0.3048) (layer F.Cu) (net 8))
 (segment (start 139.65962 120.36578) (end 148.1864 120.36578) (width 0.3048) (layer F.Cu) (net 8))
 (segment (start 137.51078 122.51462) (end 139.65962 120.36578) (width 0.3048) (layer F.Cu) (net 8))
 (segment (start 137.51078 124.46534) (end 137.51078 122.51462) (width 0.3048) (layer F.Cu) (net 8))
 (segment (start 136.26 125.82) (end 136.26 125.44) (width 0.3048) (layer F.Cu) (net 8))
 (segment (start 136.26 125.82) (end 136.26 125.19) (width 0.3048) (layer F.Cu) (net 8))
 (segment (start 136.26 125.82) (end 136.58 125.82) (width 0.3048) (layer F.Cu) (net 8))
 (segment (start 136.271 125.857) (end 136.3782 125.857) (width 0.2032) (layer B.Cu) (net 8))
 (segment (start 136.271 125.857) (end 136.556 125.857) (width 0.2032) (layer B.Cu) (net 8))
 (segment (start 135.76 125.857) (end 135.943 125.857) (width 0.2032) (layer B.Cu) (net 8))
 (segment (start 136.271 125.857) (end 136.271 125.829) (width 0.3048) (layer F.Cu) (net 8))
 (segment (start 136.271 125.857) (end 136.7338 125.857) (width 0.2032) (layer F.Cu) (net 8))
 (segment (start 136.271 125.857) (end 136.3274 125.857) (width 0.2032) (layer F.Cu) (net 8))
 (segment (start 152.73 115.23) (end 152.42 115.23) (width 0.3048) (layer B.Cu) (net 8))
 (segment (start 152.73 115.23) (end 152.73 115.47) (width 0.3048) (layer F.Cu) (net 8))
 (segment (start 133.72 123.28) (end 133.97 123.28) (width 0.3048) (layer F.Cu) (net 9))
 (segment (start 133.97 123.28) (end 135.396 121.854) (width 0.3048) (layer F.Cu) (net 9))
 (segment (start 148.9 116.52) (end 150.19 115.23) (width 0.3048) (layer F.Cu) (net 9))
 (segment (start 148.9 118.55) (end 148.9 116.52) (width 0.3048) (layer F.Cu) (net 9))
 (segment (start 147.823 119.627) (end 148.9 118.55) (width 0.3048) (layer F.Cu) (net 9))
 (segment (start 139.073 119.627) (end 147.823 119.627) (width 0.3048) (layer F.Cu) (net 9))
 (segment (start 136.846 121.854) (end 139.073 119.627) (width 0.3048) (layer F.Cu) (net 9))
 (segment (start 135.396 121.854) (end 136.846 121.854) (width 0.3048) (layer F.Cu) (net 9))
 (segment (start 133.72 123.28) (end 133.72 123.08) (width 0.3048) (layer F.Cu) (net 9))
 (segment (start 133.72 123.28) (end 133.87 123.28) (width 0.3048) (layer F.Cu) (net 9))
 (segment (start 167.97 115.23) (end 167.97 115.28) (width 0.3048) (layer B.Cu) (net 10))
 (segment (start 167.97 115.28) (end 166.7 116.55) (width 0.3048) (layer B.Cu) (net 10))
 (segment (start 133.72 127.304) (end 133.72 125.82) (width 0.3048) (layer B.Cu) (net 10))
 (segment (start 135.281 128.865) (end 133.72 127.304) (width 0.3048) (layer B.Cu) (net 10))
 (segment (start 161.107 128.865) (end 135.281 128.865) (width 0.3048) (layer B.Cu) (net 10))
 (segment (start 166.7 123.272) (end 161.107 128.865) (width 0.3048) (layer B.Cu) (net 10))
 (segment (start 166.7 116.55) (end 166.7 123.272) (width 0.3048) (layer B.Cu) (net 10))
 (segment (start 133.72 125.82) (end 133.78 125.82) (width 0.3048) (layer F.Cu) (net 10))
 (segment (start 167.97 115.23) (end 167.97 115.53) (width 0.3048) (layer F.Cu) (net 10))
 (segment (start 154.58 125.92) (end 154.57 125.92) (width 0.3048) (layer F.Cu) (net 16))
 (segment (start 154.58 125.92) (end 154.58 125.77) (width 0.3048) (layer F.Cu) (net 16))
 (segment (start 154.559 125.857) (end 154.559 125.8118) (width 0.2032) (layer B.Cu) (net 16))
 (segment (start 154.559 125.857) (end 154.559 125.6086) (width 0.3048) (layer F.Cu) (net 16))
 (segment (start 154.559 125.857) (end 154.559 125.691) (width 0.2032) (layer F.Cu) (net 16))
 (segment (start 152.04 125.92) (end 151.82 125.92) (width 0.3048) (layer F.Cu) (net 18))
 (segment (start 152.04 125.92) (end 152.04 125.81) (width 0.3048) (layer F.Cu) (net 18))
 (segment (start 156.845 125.857) (end 156.8506 125.857) (width 0.2032) (layer B.Cu) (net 13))
 (segment (start 156.845 123.317) (end 156.845 122.713) (width 0.508) (layer B.Cu) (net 14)))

